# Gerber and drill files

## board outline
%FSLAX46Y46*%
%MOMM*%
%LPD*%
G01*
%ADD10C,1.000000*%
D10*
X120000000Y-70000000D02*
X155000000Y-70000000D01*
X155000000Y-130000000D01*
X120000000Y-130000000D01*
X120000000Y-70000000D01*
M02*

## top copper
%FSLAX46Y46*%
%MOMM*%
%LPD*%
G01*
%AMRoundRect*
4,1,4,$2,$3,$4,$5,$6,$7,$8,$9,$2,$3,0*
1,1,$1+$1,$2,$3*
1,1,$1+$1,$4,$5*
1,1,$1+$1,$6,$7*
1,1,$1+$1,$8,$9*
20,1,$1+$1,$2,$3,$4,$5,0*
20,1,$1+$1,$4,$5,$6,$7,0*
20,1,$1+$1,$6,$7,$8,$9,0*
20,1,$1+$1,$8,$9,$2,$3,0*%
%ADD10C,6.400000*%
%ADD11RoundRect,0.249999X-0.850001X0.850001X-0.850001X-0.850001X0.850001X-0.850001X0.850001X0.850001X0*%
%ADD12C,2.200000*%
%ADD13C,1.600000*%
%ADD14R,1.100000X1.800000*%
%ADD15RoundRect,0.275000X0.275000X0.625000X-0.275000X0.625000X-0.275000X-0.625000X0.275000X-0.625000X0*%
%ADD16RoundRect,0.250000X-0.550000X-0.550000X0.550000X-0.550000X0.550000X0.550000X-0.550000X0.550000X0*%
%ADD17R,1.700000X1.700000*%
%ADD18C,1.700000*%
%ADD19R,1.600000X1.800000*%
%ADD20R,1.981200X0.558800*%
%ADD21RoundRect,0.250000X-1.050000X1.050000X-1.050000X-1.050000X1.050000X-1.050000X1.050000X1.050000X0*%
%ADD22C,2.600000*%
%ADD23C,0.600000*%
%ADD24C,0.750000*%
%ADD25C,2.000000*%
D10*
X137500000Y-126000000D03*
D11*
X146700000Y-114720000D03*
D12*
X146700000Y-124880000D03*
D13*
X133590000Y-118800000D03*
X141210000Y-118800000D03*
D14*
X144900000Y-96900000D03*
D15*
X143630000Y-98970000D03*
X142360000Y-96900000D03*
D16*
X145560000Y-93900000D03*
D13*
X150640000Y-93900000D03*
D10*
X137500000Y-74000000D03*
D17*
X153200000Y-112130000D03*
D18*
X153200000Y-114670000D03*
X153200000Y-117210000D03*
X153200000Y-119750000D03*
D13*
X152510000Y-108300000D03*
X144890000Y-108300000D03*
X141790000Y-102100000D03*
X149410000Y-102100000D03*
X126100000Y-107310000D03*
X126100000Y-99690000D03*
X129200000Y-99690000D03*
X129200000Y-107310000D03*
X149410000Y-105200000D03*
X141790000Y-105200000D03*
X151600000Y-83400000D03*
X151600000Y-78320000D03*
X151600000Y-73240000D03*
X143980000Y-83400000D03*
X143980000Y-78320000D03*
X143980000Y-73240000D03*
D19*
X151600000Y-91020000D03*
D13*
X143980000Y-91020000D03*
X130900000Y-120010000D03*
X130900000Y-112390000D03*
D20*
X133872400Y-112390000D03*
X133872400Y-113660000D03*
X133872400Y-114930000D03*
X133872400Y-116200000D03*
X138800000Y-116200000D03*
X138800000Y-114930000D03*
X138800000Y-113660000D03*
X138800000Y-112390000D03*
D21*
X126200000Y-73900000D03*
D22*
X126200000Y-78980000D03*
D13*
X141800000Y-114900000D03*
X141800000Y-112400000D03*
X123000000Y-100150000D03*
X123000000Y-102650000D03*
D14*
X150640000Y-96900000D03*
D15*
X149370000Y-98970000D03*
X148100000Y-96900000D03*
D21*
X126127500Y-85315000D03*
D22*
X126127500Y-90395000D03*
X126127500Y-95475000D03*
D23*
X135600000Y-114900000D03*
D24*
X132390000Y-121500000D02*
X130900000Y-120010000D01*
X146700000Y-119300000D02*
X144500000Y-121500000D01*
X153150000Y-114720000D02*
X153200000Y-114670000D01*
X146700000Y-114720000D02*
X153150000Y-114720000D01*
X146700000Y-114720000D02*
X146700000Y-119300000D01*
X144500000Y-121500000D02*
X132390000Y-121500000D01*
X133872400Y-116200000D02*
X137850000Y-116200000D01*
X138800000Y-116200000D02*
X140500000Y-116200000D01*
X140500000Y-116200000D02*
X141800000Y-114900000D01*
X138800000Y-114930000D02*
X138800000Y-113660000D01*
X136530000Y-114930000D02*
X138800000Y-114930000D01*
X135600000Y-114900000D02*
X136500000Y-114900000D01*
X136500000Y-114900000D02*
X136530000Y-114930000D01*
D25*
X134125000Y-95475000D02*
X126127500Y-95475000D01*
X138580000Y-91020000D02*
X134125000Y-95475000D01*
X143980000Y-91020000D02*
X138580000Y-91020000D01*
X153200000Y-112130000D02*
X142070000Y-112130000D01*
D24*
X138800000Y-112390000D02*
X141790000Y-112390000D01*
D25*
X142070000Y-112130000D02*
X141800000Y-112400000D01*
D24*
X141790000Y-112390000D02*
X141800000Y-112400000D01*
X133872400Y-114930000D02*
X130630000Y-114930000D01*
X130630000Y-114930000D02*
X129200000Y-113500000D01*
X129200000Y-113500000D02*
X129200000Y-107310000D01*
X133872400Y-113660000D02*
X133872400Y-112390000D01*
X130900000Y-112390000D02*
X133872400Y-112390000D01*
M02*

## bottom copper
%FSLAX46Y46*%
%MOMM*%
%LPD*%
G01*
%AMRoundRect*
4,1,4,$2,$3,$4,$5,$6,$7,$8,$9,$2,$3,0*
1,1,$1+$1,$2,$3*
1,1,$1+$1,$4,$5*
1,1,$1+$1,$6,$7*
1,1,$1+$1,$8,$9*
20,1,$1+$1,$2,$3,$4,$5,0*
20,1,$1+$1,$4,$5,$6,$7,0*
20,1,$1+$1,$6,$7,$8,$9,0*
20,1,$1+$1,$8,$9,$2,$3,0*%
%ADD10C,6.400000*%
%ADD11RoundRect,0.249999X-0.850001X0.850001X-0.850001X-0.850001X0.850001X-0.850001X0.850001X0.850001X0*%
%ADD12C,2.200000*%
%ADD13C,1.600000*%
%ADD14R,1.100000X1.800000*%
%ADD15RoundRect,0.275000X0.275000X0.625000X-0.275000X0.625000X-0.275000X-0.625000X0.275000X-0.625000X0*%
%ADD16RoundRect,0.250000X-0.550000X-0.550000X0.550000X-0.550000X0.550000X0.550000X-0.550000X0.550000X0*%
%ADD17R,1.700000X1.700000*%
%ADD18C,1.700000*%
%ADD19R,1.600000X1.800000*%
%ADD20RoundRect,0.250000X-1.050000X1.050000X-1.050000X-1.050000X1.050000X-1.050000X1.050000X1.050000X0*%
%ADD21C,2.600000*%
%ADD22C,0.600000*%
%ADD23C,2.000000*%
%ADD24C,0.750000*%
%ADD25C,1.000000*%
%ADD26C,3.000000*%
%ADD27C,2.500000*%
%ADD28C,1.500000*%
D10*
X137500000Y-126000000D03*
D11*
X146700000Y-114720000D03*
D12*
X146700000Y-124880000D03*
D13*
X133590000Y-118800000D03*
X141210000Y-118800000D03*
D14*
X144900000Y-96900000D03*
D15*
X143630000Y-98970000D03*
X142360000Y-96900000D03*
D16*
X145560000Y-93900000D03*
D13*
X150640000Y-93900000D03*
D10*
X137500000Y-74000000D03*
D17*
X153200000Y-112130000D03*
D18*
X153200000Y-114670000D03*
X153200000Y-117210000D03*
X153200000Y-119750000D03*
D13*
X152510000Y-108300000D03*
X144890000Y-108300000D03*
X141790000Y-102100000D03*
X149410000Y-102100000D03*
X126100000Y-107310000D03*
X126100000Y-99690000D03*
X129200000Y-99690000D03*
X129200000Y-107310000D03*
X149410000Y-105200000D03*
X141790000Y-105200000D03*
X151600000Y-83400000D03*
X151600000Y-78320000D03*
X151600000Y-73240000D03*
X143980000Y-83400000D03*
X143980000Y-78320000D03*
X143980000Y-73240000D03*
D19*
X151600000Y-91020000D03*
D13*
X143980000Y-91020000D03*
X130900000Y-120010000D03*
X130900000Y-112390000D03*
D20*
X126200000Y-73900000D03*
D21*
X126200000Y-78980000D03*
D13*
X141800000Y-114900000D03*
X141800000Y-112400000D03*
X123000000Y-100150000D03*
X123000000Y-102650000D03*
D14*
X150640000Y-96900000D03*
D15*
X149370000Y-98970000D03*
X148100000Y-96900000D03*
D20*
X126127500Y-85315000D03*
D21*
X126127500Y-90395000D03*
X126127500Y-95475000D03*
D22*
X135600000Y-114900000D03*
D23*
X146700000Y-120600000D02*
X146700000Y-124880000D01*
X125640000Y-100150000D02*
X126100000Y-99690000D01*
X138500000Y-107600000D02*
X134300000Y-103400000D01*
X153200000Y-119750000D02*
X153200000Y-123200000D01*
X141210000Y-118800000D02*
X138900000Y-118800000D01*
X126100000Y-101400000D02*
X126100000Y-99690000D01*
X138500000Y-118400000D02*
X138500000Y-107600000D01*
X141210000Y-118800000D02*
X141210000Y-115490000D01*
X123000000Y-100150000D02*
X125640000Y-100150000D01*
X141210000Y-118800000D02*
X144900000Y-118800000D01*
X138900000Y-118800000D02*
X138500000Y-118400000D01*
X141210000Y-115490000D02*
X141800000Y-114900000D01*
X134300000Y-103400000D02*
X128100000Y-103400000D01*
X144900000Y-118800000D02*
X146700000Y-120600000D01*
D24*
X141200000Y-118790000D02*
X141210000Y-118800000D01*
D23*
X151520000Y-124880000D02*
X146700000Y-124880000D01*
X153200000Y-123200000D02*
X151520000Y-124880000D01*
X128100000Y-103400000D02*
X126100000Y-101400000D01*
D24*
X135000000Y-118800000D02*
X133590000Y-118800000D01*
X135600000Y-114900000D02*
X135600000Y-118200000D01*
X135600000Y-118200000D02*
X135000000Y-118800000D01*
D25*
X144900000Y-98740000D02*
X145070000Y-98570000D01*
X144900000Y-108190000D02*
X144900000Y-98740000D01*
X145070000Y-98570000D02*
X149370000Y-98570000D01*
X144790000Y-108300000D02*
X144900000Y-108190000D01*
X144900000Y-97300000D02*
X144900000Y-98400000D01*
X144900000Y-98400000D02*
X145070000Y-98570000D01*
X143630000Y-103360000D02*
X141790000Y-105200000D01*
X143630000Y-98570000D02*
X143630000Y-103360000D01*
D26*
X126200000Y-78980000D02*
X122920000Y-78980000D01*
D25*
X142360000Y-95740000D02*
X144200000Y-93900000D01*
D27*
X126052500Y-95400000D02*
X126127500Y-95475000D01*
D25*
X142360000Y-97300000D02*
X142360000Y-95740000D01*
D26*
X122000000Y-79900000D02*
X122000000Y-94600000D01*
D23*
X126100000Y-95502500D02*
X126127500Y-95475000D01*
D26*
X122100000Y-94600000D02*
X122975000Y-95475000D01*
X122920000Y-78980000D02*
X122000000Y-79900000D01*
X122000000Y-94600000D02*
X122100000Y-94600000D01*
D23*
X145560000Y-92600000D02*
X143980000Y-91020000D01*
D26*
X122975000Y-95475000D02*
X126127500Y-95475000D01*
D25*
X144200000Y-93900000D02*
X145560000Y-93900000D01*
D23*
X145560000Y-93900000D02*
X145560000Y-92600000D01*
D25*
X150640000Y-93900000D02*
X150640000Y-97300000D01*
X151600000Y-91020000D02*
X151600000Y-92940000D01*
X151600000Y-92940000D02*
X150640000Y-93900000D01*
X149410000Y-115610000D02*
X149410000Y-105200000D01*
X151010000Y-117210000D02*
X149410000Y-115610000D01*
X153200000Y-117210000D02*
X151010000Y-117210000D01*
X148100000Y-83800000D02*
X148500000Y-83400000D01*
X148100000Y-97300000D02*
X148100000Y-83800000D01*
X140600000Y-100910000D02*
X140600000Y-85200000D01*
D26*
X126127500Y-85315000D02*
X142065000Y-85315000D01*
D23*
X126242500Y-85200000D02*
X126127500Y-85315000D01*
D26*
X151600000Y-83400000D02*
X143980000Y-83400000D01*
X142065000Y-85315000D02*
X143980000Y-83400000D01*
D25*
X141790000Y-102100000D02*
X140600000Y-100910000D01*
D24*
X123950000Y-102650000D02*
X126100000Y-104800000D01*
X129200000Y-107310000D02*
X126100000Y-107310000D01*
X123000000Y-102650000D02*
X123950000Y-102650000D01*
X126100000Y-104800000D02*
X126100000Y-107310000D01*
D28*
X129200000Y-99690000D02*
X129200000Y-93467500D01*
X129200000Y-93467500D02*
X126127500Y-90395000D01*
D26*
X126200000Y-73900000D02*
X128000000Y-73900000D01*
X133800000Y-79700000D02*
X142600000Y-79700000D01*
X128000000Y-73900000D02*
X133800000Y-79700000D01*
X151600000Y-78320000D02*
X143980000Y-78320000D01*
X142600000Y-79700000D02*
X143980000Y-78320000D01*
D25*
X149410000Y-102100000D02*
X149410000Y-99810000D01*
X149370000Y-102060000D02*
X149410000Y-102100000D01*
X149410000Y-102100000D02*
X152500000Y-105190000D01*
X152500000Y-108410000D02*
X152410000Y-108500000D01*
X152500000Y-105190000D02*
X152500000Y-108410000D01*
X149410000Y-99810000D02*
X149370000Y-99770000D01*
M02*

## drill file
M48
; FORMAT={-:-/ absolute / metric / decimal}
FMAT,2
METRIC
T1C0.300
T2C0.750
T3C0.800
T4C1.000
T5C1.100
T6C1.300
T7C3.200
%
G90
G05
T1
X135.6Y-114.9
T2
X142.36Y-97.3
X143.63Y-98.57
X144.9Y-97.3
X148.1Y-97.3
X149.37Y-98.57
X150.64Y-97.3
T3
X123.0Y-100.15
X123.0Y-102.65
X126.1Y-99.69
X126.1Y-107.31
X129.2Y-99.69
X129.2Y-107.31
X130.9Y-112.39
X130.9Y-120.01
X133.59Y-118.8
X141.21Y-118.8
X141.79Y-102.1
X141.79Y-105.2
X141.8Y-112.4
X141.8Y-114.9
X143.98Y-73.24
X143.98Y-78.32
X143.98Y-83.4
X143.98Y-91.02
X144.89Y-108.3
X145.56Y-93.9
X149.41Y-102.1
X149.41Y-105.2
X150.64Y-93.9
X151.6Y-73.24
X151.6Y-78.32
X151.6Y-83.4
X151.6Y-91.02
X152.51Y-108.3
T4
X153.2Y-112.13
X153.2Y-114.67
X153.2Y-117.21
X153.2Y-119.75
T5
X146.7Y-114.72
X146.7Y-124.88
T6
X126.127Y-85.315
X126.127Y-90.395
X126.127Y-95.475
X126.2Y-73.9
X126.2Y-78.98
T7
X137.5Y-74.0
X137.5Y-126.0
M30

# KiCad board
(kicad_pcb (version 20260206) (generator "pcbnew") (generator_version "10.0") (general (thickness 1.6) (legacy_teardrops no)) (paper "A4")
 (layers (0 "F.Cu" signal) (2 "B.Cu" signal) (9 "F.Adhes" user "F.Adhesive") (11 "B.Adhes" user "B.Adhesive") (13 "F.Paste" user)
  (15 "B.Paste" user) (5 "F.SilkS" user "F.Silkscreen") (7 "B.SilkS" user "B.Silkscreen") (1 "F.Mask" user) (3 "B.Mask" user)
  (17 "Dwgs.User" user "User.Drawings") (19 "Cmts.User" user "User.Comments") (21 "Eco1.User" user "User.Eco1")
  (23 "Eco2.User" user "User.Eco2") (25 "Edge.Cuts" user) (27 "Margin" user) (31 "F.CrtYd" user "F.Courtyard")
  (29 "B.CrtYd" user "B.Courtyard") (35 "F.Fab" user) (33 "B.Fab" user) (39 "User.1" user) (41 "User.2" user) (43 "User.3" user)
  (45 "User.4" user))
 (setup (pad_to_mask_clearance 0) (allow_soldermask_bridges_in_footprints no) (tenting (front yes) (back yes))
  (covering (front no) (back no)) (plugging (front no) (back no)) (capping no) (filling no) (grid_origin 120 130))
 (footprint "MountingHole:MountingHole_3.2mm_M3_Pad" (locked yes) (layer "F.Cu") (at 137.5 126)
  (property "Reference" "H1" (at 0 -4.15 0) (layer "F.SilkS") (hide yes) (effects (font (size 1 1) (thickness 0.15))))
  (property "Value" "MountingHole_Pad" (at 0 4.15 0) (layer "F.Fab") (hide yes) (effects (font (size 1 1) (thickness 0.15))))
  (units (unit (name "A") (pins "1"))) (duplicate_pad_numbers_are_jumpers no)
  (pad "1" thru_hole circle (at 0 0) (size 6.4 6.4) (drill 3.2) (layers "*.Cu" "*.Mask") (remove_unused_layers no)
   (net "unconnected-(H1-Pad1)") (zone_connect 2)))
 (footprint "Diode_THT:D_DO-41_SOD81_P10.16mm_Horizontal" (layer "F.Cu") (at 146.7 114.72 -90)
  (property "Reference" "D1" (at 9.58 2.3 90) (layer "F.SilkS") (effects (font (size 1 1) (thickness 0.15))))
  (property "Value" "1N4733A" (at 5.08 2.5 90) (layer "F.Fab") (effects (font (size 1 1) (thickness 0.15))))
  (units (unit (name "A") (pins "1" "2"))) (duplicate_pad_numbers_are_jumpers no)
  (pad "1" thru_hole roundrect (at 0 0 270) (size 2.2 2.2) (drill 1.1) (layers "*.Cu" "*.Mask") (remove_unused_layers no)
   (roundrect_rratio 0.113636) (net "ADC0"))
  (pad "2" thru_hole circle (at 10.16 0 270) (size 2.2 2.2) (drill 1.1) (layers "*.Cu" "*.Mask") (remove_unused_layers no) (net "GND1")))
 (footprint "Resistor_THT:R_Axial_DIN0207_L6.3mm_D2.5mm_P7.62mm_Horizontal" (layer "F.Cu") (at 133.59 118.8)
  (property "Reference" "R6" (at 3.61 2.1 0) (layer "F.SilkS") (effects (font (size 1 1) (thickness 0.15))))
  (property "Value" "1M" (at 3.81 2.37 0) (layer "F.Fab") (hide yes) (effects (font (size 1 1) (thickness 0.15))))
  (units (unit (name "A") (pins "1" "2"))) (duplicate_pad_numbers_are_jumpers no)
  (pad "1" thru_hole circle (at 0 0) (size 1.6 1.6) (drill 0.8) (layers "*.Cu" "*.Mask") (remove_unused_layers no) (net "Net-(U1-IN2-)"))
  (pad "2" thru_hole circle (at 7.62 0) (size 1.6 1.6) (drill 0.8) (layers "*.Cu" "*.Mask") (remove_unused_layers no) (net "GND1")))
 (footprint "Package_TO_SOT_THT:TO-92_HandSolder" (layer "F.Cu") (at 144.9 97.3 180)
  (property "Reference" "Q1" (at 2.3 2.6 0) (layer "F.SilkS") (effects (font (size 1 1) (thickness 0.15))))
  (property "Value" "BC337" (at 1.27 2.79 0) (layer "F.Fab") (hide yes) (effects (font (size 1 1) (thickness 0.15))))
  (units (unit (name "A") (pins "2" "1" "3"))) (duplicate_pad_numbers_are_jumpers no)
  (pad "1" thru_hole rect (at 0 0 180) (size 1.1 1.8) (drill 0.75 (offset 0 0.4)) (layers "*.Cu" "*.Mask") (remove_unused_layers no)
   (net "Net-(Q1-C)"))
  (pad "2" thru_hole roundrect (at 1.27 -1.27 180) (size 1.1 1.8) (drill 0.75 (offset 0 -0.4)) (layers "*.Cu" "*.Mask")
   (remove_unused_layers no) (roundrect_rratio 0.25) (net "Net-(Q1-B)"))
  (pad "3" thru_hole roundrect (at 2.54 0 180) (size 1.1 1.8) (drill 0.75 (offset 0 0.4)) (layers "*.Cu" "*.Mask") (remove_unused_layers no)
   (roundrect_rratio 0.25) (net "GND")))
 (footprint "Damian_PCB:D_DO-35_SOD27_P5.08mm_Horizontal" (layer "F.Cu") (at 148.1 93.9)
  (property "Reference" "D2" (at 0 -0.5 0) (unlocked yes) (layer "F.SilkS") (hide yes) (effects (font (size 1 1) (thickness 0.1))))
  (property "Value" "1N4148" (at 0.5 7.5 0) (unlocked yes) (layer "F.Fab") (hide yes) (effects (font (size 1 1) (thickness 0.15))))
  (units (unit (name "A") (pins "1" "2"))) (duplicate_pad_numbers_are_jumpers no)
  (pad "1" thru_hole roundrect (at -2.54 0) (size 1.6 1.6) (drill 0.8) (layers "*.Cu" "*.Mask") (remove_unused_layers no)
   (roundrect_rratio 0.15625) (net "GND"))
  (pad "2" thru_hole circle (at 2.54 0) (size 1.6 1.6) (drill 0.8) (layers "*.Cu" "*.Mask") (remove_unused_layers no) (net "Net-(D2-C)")))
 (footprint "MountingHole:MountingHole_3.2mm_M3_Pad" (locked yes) (layer "F.Cu") (at 137.5 74)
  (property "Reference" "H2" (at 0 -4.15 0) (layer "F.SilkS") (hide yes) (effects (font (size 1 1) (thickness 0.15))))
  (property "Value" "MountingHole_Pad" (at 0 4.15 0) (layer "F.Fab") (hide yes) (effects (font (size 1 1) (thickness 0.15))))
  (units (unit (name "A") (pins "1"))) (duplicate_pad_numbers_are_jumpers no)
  (pad "1" thru_hole circle (at 0 0) (size 6.4 6.4) (drill 3.2) (layers "*.Cu" "*.Mask") (remove_unused_layers no)
   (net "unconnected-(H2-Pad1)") (zone_connect 2)))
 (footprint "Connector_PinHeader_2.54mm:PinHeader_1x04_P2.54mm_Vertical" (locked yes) (layer "F.Cu") (at 153.2 112.13)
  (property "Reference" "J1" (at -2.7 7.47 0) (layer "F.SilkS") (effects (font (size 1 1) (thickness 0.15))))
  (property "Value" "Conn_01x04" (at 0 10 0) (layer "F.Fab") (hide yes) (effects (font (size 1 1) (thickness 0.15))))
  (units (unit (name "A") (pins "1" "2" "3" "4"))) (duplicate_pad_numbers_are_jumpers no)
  (pad "1" thru_hole rect (at 0 0) (size 1.7 1.7) (drill 1) (layers "*.Cu" "*.Mask") (remove_unused_layers no) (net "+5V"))
  (pad "2" thru_hole circle (at 0 2.54) (size 1.7 1.7) (drill 1) (layers "*.Cu" "*.Mask") (remove_unused_layers no) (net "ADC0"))
  (pad "3" thru_hole circle (at 0 5.08) (size 1.7 1.7) (drill 1) (layers "*.Cu" "*.Mask") (remove_unused_layers no) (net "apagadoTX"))
  (pad "4" thru_hole circle (at 0 7.62) (size 1.7 1.7) (drill 1) (layers "*.Cu" "*.Mask") (remove_unused_layers no) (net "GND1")))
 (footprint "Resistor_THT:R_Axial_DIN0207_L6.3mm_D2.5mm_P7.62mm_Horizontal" (layer "F.Cu") (at 152.51 108.3 180)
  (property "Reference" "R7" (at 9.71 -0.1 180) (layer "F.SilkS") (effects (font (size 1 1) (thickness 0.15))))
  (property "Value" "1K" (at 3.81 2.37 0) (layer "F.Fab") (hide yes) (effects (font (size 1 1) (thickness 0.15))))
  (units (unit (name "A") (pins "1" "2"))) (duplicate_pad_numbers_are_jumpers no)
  (pad "1" thru_hole circle (at 0 0 180) (size 1.6 1.6) (drill 0.8) (layers "*.Cu" "*.Mask") (remove_unused_layers no) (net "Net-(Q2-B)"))
  (pad "2" thru_hole circle (at 7.62 0 180) (size 1.6 1.6) (drill 0.8) (layers "*.Cu" "*.Mask") (remove_unused_layers no) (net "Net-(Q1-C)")))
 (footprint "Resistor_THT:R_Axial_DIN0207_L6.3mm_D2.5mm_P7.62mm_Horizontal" (layer "F.Cu") (at 141.79 102.1)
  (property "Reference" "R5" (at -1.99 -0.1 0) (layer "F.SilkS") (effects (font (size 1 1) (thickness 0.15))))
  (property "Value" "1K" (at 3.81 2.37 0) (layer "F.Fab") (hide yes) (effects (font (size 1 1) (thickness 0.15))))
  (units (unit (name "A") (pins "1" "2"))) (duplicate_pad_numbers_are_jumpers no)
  (pad "1" thru_hole circle (at 0 0) (size 1.6 1.6) (drill 0.8) (layers "*.Cu" "*.Mask") (remove_unused_layers no) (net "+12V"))
  (pad "2" thru_hole circle (at 7.62 0) (size 1.6 1.6) (drill 0.8) (layers "*.Cu" "*.Mask") (remove_unused_layers no) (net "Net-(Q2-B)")))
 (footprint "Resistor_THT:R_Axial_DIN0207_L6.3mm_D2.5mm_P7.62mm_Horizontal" (layer "F.Cu") (at 126.1 107.31 90)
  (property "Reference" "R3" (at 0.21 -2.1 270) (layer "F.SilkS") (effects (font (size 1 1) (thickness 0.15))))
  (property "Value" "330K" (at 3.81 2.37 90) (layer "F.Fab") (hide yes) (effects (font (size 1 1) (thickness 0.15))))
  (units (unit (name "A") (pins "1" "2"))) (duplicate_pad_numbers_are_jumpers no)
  (pad "1" thru_hole circle (at 0 0 90) (size 1.6 1.6) (drill 0.8) (layers "*.Cu" "*.Mask") (remove_unused_layers no) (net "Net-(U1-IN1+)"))
  (pad "2" thru_hole circle (at 7.62 0 90) (size 1.6 1.6) (drill 0.8) (layers "*.Cu" "*.Mask") (remove_unused_layers no) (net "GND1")))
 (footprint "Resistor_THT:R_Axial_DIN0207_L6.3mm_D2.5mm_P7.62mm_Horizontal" (layer "F.Cu") (at 129.2 99.69 -90)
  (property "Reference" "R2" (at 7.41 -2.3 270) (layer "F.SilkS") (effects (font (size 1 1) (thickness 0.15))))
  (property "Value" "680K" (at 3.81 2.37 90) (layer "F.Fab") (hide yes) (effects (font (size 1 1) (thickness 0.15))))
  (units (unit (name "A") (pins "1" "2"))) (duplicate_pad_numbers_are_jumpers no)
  (pad "1" thru_hole circle (at 0 0 270) (size 1.6 1.6) (drill 0.8) (layers "*.Cu" "*.Mask") (remove_unused_layers no) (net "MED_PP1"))
  (pad "2" thru_hole circle (at 7.62 0 270) (size 1.6 1.6) (drill 0.8) (layers "*.Cu" "*.Mask") (remove_unused_layers no)
   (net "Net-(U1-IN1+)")))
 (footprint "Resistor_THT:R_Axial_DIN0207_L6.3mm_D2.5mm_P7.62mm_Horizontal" (layer "F.Cu") (at 149.41 105.2 180)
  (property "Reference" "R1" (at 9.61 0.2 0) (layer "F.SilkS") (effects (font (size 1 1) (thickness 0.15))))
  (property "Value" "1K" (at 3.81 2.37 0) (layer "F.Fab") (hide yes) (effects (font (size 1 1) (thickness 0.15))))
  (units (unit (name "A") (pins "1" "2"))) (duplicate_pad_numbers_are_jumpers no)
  (pad "1" thru_hole circle (at 0 0 180) (size 1.6 1.6) (drill 0.8) (layers "*.Cu" "*.Mask") (remove_unused_layers no) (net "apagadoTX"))
  (pad "2" thru_hole circle (at 7.62 0 180) (size 1.6 1.6) (drill 0.8) (layers "*.Cu" "*.Mask") (remove_unused_layers no) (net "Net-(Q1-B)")))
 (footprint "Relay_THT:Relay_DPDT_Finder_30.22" (layer "F.Cu") (at 151.6 91.02 90)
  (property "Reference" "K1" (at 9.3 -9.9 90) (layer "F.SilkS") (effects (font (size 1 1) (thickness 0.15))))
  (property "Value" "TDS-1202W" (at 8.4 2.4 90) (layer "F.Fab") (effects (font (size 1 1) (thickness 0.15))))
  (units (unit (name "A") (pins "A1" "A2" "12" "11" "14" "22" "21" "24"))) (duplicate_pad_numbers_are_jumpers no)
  (pad "11" thru_hole circle (at 7.62 0 180) (size 1.6 1.6) (drill 0.8) (layers "*.Cu" "*.Mask") (remove_unused_layers no) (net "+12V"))
  (pad "12" thru_hole circle (at 12.7 0 180) (size 1.6 1.6) (drill 0.8) (layers "*.Cu" "*.Mask") (remove_unused_layers no) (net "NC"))
  (pad "14" thru_hole circle (at 17.78 0 180) (size 1.6 1.6) (drill 0.8) (layers "*.Cu" "*.Mask") (remove_unused_layers no)
   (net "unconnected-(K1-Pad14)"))
  (pad "21" thru_hole circle (at 7.62 -7.62 180) (size 1.6 1.6) (drill 0.8) (layers "*.Cu" "*.Mask") (remove_unused_layers no) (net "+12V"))
  (pad "22" thru_hole circle (at 12.7 -7.62 180) (size 1.6 1.6) (drill 0.8) (layers "*.Cu" "*.Mask") (remove_unused_layers no) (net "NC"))
  (pad "24" thru_hole circle (at 17.78 -7.62 270) (size 1.6 1.6) (drill 0.8) (layers "*.Cu" "*.Mask") (remove_unused_layers no)
   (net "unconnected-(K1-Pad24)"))
  (pad "A1" thru_hole rect (at 0 0 180) (size 1.6 1.8) (drill 0.8) (layers "*.Cu" "*.Mask") (remove_unused_layers no) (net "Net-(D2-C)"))
  (pad "A2" thru_hole circle (at 0 -7.62 180) (size 1.6 1.6) (drill 0.8) (layers "*.Cu" "*.Mask") (remove_unused_layers no) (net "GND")))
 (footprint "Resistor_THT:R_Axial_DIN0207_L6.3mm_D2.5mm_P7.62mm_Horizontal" (layer "F.Cu") (at 130.9 120.01 90)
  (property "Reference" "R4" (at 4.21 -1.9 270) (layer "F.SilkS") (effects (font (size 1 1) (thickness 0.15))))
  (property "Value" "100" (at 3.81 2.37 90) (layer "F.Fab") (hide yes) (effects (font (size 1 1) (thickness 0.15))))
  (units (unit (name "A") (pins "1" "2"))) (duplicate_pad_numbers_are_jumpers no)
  (pad "1" thru_hole circle (at 0 0 90) (size 1.6 1.6) (drill 0.8) (layers "*.Cu" "*.Mask") (remove_unused_layers no) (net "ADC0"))
  (pad "2" thru_hole circle (at 7.62 0 90) (size 1.6 1.6) (drill 0.8) (layers "*.Cu" "*.Mask") (remove_unused_layers no)
   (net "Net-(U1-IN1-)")))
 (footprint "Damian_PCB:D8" (layer "F.Cu") (at 136.3362 114.295)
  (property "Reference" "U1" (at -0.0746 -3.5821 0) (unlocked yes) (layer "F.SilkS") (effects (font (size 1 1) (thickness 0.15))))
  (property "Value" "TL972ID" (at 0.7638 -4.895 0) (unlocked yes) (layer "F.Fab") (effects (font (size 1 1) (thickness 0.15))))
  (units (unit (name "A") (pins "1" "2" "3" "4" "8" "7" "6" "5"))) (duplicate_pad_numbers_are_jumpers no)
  (pad "1" smd rect (at -2.4638 -1.905) (size 1.9812 0.5588) (layers "F.Cu" "F.Mask" "F.Paste") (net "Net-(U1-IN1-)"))
  (pad "2" smd rect (at -2.4638 -0.635) (size 1.9812 0.5588) (layers "F.Cu" "F.Mask" "F.Paste") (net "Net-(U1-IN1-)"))
  (pad "3" smd rect (at -2.4638 0.635) (size 1.9812 0.5588) (layers "F.Cu" "F.Mask" "F.Paste") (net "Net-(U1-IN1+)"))
  (pad "4" smd rect (at -2.4638 1.905) (size 1.9812 0.5588) (layers "F.Cu" "F.Mask" "F.Paste") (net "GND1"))
  (pad "5" smd rect (at 2.4638 1.905) (size 1.9812 0.5588) (layers "F.Cu" "F.Mask" "F.Paste") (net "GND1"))
  (pad "6" smd rect (at 2.4638 0.635) (size 1.9812 0.5588) (layers "F.Cu" "F.Mask" "F.Paste") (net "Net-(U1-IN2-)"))
  (pad "7" smd rect (at 2.4638 -0.635) (size 1.9812 0.5588) (layers "F.Cu" "F.Mask" "F.Paste") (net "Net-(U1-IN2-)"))
  (pad "8" smd rect (at 2.4638 -1.905) (size 1.9812 0.5588) (layers "F.Cu" "F.Mask" "F.Paste") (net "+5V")))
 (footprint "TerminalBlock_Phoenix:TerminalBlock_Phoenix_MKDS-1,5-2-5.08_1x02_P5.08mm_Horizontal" (layer "F.Cu") (at 126.2 73.9 -90)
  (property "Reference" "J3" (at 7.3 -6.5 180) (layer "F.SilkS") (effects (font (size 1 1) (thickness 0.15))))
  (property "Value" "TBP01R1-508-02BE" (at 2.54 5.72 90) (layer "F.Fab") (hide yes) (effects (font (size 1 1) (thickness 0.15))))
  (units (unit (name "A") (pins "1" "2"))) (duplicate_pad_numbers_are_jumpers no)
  (pad "1" thru_hole roundrect (at 0 0 270) (size 2.6 2.6) (drill 1.3) (layers "*.Cu" "*.Mask") (remove_unused_layers no)
   (roundrect_rratio 0.096154) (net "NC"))
  (pad "2" thru_hole circle (at 5.08 0 270) (size 2.6 2.6) (drill 1.3) (layers "*.Cu" "*.Mask") (remove_unused_layers no) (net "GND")))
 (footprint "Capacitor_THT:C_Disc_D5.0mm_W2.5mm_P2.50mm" (layer "F.Cu") (at 141.8 114.9 90)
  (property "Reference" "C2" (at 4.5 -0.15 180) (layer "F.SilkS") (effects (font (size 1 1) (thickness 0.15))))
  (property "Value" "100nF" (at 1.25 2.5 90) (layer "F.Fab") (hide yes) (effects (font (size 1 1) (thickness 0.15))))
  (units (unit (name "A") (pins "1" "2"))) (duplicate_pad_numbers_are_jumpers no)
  (pad "1" thru_hole circle (at 0 0 90) (size 1.6 1.6) (drill 0.8) (layers "*.Cu" "*.Mask") (remove_unused_layers no) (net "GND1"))
  (pad "2" thru_hole circle (at 2.5 0 90) (size 1.6 1.6) (drill 0.8) (layers "*.Cu" "*.Mask") (remove_unused_layers no) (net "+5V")))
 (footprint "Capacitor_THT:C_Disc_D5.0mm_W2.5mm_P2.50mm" (layer "F.Cu") (at 123 100.15 -90)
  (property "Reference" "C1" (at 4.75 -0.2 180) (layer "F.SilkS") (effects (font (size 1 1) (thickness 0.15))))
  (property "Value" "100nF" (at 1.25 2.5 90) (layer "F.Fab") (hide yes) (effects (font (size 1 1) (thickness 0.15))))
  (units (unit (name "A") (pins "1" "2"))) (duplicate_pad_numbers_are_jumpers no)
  (pad "1" thru_hole circle (at 0 0 270) (size 1.6 1.6) (drill 0.8) (layers "*.Cu" "*.Mask") (remove_unused_layers no) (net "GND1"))
  (pad "2" thru_hole circle (at 2.5 0 270) (size 1.6 1.6) (drill 0.8) (layers "*.Cu" "*.Mask") (remove_unused_layers no)
   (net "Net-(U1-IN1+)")))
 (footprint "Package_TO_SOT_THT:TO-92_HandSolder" (layer "F.Cu") (at 150.64 97.3 180)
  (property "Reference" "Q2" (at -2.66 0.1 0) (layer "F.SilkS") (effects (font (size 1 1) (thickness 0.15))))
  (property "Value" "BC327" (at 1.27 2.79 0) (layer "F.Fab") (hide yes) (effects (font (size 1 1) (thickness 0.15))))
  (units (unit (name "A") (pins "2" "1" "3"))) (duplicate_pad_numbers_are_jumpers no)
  (pad "1" thru_hole rect (at 0 0 180) (size 1.1 1.8) (drill 0.75 (offset 0 0.4)) (layers "*.Cu" "*.Mask") (remove_unused_layers no)
   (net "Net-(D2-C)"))
  (pad "2" thru_hole roundrect (at 1.27 -1.27 180) (size 1.1 1.8) (drill 0.75 (offset 0 -0.4)) (layers "*.Cu" "*.Mask")
   (remove_unused_layers no) (roundrect_rratio 0.25) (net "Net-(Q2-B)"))
  (pad "3" thru_hole roundrect (at 2.54 0 180) (size 1.1 1.8) (drill 0.75 (offset 0 0.4)) (layers "*.Cu" "*.Mask") (remove_unused_layers no)
   (roundrect_rratio 0.25) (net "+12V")))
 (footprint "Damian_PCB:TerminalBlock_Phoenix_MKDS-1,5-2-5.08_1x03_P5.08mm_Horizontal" (layer "F.Cu") (at 126.1275 85.315 -90)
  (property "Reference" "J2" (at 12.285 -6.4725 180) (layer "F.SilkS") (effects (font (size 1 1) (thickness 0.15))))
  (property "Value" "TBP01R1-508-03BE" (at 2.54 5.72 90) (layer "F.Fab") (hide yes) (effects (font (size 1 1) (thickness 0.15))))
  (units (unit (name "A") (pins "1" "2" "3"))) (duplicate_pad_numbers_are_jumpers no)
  (pad "1" thru_hole roundrect (at 0 0 270) (size 2.6 2.6) (drill 1.3) (layers "*.Cu" "*.Mask") (remove_unused_layers no)
   (roundrect_rratio 0.096154) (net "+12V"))
  (pad "2" thru_hole circle (at 5.08 0 270) (size 2.6 2.6) (drill 1.3) (layers "*.Cu" "*.Mask") (remove_unused_layers no) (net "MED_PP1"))
  (pad "3" thru_hole circle (at 10.16 0 270) (size 2.6 2.6) (drill 1.3) (layers "*.Cu" "*.Mask") (remove_unused_layers no) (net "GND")))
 (gr_rect (start 120 70) (end 155 130) (stroke (width 1) (type solid)) (fill no) (locked yes) (layer "Edge.Cuts"))
 (segment (start 132.39 121.5) (end 130.9 120.01) (width 0.75) (layer "F.Cu") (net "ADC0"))
 (segment (start 146.7 119.3) (end 144.5 121.5) (width 0.75) (layer "F.Cu") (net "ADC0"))
 (segment (start 153.15 114.72) (end 153.2 114.67) (width 0.75) (layer "F.Cu") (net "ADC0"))
 (segment (start 146.7 114.72) (end 153.15 114.72) (width 0.75) (layer "F.Cu") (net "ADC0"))
 (segment (start 146.7 114.72) (end 146.7 119.3) (width 0.75) (layer "F.Cu") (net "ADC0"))
 (segment (start 144.5 121.5) (end 132.39 121.5) (width 0.75) (layer "F.Cu") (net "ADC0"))
 (segment (start 133.8724 116.2) (end 137.85 116.2) (width 0.75) (layer "F.Cu") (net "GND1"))
 (segment (start 138.8 116.2) (end 140.5 116.2) (width 0.75) (layer "F.Cu") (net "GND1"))
 (segment (start 140.5 116.2) (end 141.8 114.9) (width 0.75) (layer "F.Cu") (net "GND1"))
 (segment (start 146.7 120.6) (end 146.7 124.88) (width 2) (layer "B.Cu") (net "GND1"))
 (segment (start 125.64 100.15) (end 126.1 99.69) (width 2) (layer "B.Cu") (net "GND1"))
 (segment (start 138.5 107.6) (end 134.3 103.4) (width 2) (layer "B.Cu") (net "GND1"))
 (segment (start 153.2 119.75) (end 153.2 123.2) (width 2) (layer "B.Cu") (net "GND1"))
 (segment (start 141.21 118.8) (end 138.9 118.8) (width 2) (layer "B.Cu") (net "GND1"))
 (segment (start 126.1 101.4) (end 126.1 99.69) (width 2) (layer "B.Cu") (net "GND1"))
 (segment (start 138.5 118.4) (end 138.5 107.6) (width 2) (layer "B.Cu") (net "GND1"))
 (segment (start 141.21 118.8) (end 141.21 115.49) (width 2) (layer "B.Cu") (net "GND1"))
 (segment (start 123 100.15) (end 125.64 100.15) (width 2) (layer "B.Cu") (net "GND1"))
 (segment (start 141.21 118.8) (end 144.9 118.8) (width 2) (layer "B.Cu") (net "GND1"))
 (segment (start 138.9 118.8) (end 138.5 118.4) (width 2) (layer "B.Cu") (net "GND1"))
 (segment (start 141.21 115.49) (end 141.8 114.9) (width 2) (layer "B.Cu") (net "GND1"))
 (segment (start 134.3 103.4) (end 128.1 103.4) (width 2) (layer "B.Cu") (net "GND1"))
 (segment (start 144.9 118.8) (end 146.7 120.6) (width 2) (layer "B.Cu") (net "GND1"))
 (segment (start 141.2 118.79) (end 141.21 118.8) (width 0.75) (layer "B.Cu") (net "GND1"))
 (segment (start 151.52 124.88) (end 146.7 124.88) (width 2) (layer "B.Cu") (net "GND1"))
 (segment (start 153.2 123.2) (end 151.52 124.88) (width 2) (layer "B.Cu") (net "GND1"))
 (segment (start 128.1 103.4) (end 126.1 101.4) (width 2) (layer "B.Cu") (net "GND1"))
 (segment (start 138.8 114.93) (end 138.8 113.66) (width 0.75) (layer "F.Cu") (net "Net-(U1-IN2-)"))
 (segment (start 136.53 114.93) (end 138.8 114.93) (width 0.75) (layer "F.Cu") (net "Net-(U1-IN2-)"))
 (segment (start 135.6 114.9) (end 136.5 114.9) (width 0.75) (layer "F.Cu") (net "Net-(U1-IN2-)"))
 (segment (start 136.5 114.9) (end 136.53 114.93) (width 0.75) (layer "F.Cu") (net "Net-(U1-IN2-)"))
 (via (at 135.6 114.9) (size 0.6) (drill 0.3) (layers "F.Cu" "B.Cu") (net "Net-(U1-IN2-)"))
 (segment (start 135 118.8) (end 133.59 118.8) (width 0.75) (layer "B.Cu") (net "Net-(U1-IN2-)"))
 (segment (start 135.6 114.9) (end 135.6 118.2) (width 0.75) (layer "B.Cu") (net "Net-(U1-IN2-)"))
 (segment (start 135.6 118.2) (end 135 118.8) (width 0.75) (layer "B.Cu") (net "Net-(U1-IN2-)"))
 (segment (start 144.9 98.74) (end 145.07 98.57) (width 1) (layer "B.Cu") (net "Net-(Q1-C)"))
 (segment (start 144.9 108.19) (end 144.9 98.74) (width 1) (layer "B.Cu") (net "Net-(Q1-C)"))
 (segment (start 145.07 98.57) (end 149.37 98.57) (width 1) (layer "B.Cu") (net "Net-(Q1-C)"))
 (segment (start 144.79 108.3) (end 144.9 108.19) (width 1) (layer "B.Cu") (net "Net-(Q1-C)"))
 (segment (start 144.9 97.3) (end 144.9 98.4) (width 1) (layer "B.Cu") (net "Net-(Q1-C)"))
 (segment (start 144.9 98.4) (end 145.07 98.57) (width 1) (layer "B.Cu") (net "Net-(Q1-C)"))
 (segment (start 143.63 103.36) (end 141.79 105.2) (width 1) (layer "B.Cu") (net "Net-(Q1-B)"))
 (segment (start 143.63 98.57) (end 143.63 103.36) (width 1) (layer "B.Cu") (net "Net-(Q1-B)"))
 (segment (start 134.125 95.475) (end 126.1275 95.475) (width 2) (layer "F.Cu") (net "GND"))
 (segment (start 138.58 91.02) (end 134.125 95.475) (width 2) (layer "F.Cu") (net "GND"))
 (segment (start 143.98 91.02) (end 138.58 91.02) (width 2) (layer "F.Cu") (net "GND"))
 (segment (start 126.2 78.98) (end 122.92 78.98) (width 3) (layer "B.Cu") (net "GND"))
 (segment (start 142.36 95.74) (end 144.2 93.9) (width 1) (layer "B.Cu") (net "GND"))
 (segment (start 126.0525 95.4) (end 126.1275 95.475) (width 2.5) (layer "B.Cu") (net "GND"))
 (segment (start 142.36 97.3) (end 142.36 95.74) (width 1) (layer "B.Cu") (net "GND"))
 (segment (start 122 79.9) (end 122 94.6) (width 3) (layer "B.Cu") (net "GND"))
 (segment (start 126.1 95.5025) (end 126.1275 95.475) (width 2) (layer "B.Cu") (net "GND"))
 (segment (start 122.1 94.6) (end 122.975 95.475) (width 3) (layer "B.Cu") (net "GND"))
 (segment (start 122.92 78.98) (end 122 79.9) (width 3) (layer "B.Cu") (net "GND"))
 (segment (start 122 94.6) (end 122.1 94.6) (width 3) (layer "B.Cu") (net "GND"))
 (segment (start 145.56 92.6) (end 143.98 91.02) (width 2) (layer "B.Cu") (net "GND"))
 (segment (start 122.975 95.475) (end 126.1275 95.475) (width 3) (layer "B.Cu") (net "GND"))
 (segment (start 144.2 93.9) (end 145.56 93.9) (width 1) (layer "B.Cu") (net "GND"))
 (segment (start 145.56 93.9) (end 145.56 92.6) (width 2) (layer "B.Cu") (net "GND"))
 (segment (start 150.64 93.9) (end 150.64 97.3) (width 1) (layer "B.Cu") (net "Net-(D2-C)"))
 (segment (start 151.6 91.02) (end 151.6 92.94) (width 1) (layer "B.Cu") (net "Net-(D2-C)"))
 (segment (start 151.6 92.94) (end 150.64 93.9) (width 1) (layer "B.Cu") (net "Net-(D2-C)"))
 (segment (start 153.2 112.13) (end 142.07 112.13) (width 2) (layer "F.Cu") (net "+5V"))
 (segment (start 138.8 112.39) (end 141.79 112.39) (width 0.75) (layer "F.Cu") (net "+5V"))
 (segment (start 142.07 112.13) (end 141.8 112.4) (width 2) (layer "F.Cu") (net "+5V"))
 (segment (start 141.79 112.39) (end 141.8 112.4) (width 0.75) (layer "F.Cu") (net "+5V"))
 (segment (start 149.41 115.61) (end 149.41 105.2) (width 1) (layer "B.Cu") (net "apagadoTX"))
 (segment (start 151.01 117.21) (end 149.41 115.61) (width 1) (layer "B.Cu") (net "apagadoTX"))
 (segment (start 153.2 117.21) (end 151.01 117.21) (width 1) (layer "B.Cu") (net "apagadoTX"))
 (segment (start 148.1 83.8) (end 148.5 83.4) (width 1) (layer "B.Cu") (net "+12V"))
 (segment (start 148.1 97.3) (end 148.1 83.8) (width 1) (layer "B.Cu") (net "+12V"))
 (segment (start 140.6 100.91) (end 140.6 85.2) (width 1) (layer "B.Cu") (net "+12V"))
 (segment (start 126.1275 85.315) (end 142.065 85.315) (width 3) (layer "B.Cu") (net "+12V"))
 (segment (start 126.2425 85.2) (end 126.1275 85.315) (width 2) (layer "B.Cu") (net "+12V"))
 (segment (start 151.6 83.4) (end 143.98 83.4) (width 3) (layer "B.Cu") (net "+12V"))
 (segment (start 142.065 85.315) (end 143.98 83.4) (width 3) (layer "B.Cu") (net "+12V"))
 (segment (start 141.79 102.1) (end 140.6 100.91) (width 1) (layer "B.Cu") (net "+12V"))
 (segment (start 133.8724 114.93) (end 130.63 114.93) (width 0.75) (layer "F.Cu") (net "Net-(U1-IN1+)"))
 (segment (start 130.63 114.93) (end 129.2 113.5) (width 0.75) (layer "F.Cu") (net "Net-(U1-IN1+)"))
 (segment (start 129.2 113.5) (end 129.2 107.31) (width 0.75) (layer "F.Cu") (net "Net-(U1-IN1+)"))
 (segment (start 123.95 102.65) (end 126.1 104.8) (width 0.75) (layer "B.Cu") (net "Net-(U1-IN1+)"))
 (segment (start 129.2 107.31) (end 126.1 107.31) (width 0.75) (layer "B.Cu") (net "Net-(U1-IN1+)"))
 (segment (start 123 102.65) (end 123.95 102.65) (width 0.75) (layer "B.Cu") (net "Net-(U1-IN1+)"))
 (segment (start 126.1 104.8) (end 126.1 107.31) (width 0.75) (layer "B.Cu") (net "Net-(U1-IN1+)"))
 (segment (start 129.2 99.69) (end 129.2 93.4675) (width 1.5) (layer "B.Cu") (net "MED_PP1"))
 (segment (start 129.2 93.4675) (end 126.1275 90.395) (width 1.5) (layer "B.Cu") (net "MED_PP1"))
 (segment (start 126.2 73.9) (end 128 73.9) (width 3) (layer "B.Cu") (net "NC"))
 (segment (start 133.8 79.7) (end 142.6 79.7) (width 3) (layer "B.Cu") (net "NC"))
 (segment (start 128 73.9) (end 133.8 79.7) (width 3) (layer "B.Cu") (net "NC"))
 (segment (start 151.6 78.32) (end 143.98 78.32) (width 3) (layer "B.Cu") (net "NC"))
 (segment (start 142.6 79.7) (end 143.98 78.32) (width 3) (layer "B.Cu") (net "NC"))
 (segment (start 133.8724 113.66) (end 133.8724 112.39) (width 0.75) (layer "F.Cu") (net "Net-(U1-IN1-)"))
 (segment (start 130.9 112.39) (end 133.8724 112.39) (width 0.75) (layer "F.Cu") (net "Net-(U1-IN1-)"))
 (segment (start 149.41 102.1) (end 149.41 99.81) (width 1) (layer "B.Cu") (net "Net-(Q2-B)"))
 (segment (start 149.37 102.06) (end 149.41 102.1) (width 1) (layer "B.Cu") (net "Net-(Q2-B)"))
 (segment (start 149.41 102.1) (end 152.5 105.19) (width 1) (layer "B.Cu") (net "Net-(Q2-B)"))
 (segment (start 152.5 108.41) (end 152.41 108.5) (width 1) (layer "B.Cu") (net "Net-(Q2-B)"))
 (segment (start 152.5 105.19) (end 152.5 108.41) (width 1) (layer "B.Cu") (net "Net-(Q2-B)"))
 (segment (start 149.41 99.81) (end 149.37 99.77) (width 1) (layer "B.Cu") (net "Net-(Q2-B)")))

